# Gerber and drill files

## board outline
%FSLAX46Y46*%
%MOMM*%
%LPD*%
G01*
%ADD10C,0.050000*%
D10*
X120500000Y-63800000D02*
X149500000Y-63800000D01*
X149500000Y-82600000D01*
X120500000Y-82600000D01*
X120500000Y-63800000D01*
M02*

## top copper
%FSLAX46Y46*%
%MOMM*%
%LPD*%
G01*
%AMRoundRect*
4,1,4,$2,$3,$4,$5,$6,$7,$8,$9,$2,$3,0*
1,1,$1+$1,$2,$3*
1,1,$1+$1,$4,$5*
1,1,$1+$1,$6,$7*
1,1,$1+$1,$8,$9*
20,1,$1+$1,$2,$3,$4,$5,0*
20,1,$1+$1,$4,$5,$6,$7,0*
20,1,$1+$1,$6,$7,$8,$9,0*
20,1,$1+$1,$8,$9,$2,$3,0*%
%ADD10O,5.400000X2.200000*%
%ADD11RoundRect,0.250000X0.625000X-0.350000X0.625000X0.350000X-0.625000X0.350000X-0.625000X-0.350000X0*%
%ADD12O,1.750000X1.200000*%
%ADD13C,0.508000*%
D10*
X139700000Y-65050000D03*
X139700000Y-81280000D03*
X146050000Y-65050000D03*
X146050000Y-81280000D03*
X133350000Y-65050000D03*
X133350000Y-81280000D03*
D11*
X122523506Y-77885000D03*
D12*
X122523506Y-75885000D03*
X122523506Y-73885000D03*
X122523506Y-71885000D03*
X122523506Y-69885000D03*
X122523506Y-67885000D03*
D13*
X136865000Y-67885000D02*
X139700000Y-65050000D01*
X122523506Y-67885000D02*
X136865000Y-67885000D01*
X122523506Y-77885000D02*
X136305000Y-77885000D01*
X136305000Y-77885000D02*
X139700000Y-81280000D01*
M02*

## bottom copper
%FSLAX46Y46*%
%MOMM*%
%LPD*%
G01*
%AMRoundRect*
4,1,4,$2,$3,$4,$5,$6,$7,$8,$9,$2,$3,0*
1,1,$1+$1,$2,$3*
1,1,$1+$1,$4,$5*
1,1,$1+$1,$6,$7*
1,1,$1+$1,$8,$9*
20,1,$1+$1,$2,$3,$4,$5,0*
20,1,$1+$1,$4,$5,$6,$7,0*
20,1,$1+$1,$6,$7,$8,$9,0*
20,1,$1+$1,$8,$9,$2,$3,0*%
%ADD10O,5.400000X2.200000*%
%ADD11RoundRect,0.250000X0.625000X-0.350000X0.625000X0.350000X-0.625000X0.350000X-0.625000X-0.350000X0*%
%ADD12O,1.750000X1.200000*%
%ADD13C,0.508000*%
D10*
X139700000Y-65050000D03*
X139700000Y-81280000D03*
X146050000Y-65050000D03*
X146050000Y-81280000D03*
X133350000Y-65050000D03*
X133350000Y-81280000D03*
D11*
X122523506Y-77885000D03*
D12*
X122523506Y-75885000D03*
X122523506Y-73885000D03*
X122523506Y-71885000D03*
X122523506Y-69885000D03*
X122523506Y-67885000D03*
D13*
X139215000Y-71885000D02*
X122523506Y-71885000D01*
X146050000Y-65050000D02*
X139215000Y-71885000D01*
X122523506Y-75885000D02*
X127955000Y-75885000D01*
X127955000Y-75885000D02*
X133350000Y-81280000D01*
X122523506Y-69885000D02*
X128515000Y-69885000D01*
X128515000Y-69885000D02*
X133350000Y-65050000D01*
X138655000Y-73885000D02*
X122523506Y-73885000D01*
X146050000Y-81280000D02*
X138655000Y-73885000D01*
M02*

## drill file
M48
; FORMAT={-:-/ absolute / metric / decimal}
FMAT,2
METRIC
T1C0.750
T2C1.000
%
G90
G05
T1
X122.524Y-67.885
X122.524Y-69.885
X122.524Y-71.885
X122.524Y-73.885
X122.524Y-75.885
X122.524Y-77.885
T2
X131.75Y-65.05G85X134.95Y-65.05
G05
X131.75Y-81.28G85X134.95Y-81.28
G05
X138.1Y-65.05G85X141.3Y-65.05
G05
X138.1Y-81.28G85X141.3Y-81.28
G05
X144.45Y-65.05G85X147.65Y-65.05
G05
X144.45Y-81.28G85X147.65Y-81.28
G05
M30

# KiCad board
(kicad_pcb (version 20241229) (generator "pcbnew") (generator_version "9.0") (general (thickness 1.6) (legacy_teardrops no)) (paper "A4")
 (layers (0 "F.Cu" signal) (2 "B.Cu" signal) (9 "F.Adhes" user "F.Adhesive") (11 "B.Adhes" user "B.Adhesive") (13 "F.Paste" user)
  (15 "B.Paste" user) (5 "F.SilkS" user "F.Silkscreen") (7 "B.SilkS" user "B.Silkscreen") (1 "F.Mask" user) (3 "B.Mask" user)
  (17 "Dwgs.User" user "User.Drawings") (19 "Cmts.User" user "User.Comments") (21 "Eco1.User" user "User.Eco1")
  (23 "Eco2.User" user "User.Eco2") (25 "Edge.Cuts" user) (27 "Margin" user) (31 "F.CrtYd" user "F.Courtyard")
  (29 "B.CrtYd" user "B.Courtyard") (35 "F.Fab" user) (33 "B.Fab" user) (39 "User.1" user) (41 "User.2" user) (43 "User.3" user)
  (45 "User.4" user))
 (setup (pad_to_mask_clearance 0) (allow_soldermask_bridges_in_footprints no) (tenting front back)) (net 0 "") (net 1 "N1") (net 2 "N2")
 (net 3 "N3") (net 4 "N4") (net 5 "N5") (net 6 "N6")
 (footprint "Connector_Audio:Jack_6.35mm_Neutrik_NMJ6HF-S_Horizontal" (layer "F.Cu") (at 133.35 65.05)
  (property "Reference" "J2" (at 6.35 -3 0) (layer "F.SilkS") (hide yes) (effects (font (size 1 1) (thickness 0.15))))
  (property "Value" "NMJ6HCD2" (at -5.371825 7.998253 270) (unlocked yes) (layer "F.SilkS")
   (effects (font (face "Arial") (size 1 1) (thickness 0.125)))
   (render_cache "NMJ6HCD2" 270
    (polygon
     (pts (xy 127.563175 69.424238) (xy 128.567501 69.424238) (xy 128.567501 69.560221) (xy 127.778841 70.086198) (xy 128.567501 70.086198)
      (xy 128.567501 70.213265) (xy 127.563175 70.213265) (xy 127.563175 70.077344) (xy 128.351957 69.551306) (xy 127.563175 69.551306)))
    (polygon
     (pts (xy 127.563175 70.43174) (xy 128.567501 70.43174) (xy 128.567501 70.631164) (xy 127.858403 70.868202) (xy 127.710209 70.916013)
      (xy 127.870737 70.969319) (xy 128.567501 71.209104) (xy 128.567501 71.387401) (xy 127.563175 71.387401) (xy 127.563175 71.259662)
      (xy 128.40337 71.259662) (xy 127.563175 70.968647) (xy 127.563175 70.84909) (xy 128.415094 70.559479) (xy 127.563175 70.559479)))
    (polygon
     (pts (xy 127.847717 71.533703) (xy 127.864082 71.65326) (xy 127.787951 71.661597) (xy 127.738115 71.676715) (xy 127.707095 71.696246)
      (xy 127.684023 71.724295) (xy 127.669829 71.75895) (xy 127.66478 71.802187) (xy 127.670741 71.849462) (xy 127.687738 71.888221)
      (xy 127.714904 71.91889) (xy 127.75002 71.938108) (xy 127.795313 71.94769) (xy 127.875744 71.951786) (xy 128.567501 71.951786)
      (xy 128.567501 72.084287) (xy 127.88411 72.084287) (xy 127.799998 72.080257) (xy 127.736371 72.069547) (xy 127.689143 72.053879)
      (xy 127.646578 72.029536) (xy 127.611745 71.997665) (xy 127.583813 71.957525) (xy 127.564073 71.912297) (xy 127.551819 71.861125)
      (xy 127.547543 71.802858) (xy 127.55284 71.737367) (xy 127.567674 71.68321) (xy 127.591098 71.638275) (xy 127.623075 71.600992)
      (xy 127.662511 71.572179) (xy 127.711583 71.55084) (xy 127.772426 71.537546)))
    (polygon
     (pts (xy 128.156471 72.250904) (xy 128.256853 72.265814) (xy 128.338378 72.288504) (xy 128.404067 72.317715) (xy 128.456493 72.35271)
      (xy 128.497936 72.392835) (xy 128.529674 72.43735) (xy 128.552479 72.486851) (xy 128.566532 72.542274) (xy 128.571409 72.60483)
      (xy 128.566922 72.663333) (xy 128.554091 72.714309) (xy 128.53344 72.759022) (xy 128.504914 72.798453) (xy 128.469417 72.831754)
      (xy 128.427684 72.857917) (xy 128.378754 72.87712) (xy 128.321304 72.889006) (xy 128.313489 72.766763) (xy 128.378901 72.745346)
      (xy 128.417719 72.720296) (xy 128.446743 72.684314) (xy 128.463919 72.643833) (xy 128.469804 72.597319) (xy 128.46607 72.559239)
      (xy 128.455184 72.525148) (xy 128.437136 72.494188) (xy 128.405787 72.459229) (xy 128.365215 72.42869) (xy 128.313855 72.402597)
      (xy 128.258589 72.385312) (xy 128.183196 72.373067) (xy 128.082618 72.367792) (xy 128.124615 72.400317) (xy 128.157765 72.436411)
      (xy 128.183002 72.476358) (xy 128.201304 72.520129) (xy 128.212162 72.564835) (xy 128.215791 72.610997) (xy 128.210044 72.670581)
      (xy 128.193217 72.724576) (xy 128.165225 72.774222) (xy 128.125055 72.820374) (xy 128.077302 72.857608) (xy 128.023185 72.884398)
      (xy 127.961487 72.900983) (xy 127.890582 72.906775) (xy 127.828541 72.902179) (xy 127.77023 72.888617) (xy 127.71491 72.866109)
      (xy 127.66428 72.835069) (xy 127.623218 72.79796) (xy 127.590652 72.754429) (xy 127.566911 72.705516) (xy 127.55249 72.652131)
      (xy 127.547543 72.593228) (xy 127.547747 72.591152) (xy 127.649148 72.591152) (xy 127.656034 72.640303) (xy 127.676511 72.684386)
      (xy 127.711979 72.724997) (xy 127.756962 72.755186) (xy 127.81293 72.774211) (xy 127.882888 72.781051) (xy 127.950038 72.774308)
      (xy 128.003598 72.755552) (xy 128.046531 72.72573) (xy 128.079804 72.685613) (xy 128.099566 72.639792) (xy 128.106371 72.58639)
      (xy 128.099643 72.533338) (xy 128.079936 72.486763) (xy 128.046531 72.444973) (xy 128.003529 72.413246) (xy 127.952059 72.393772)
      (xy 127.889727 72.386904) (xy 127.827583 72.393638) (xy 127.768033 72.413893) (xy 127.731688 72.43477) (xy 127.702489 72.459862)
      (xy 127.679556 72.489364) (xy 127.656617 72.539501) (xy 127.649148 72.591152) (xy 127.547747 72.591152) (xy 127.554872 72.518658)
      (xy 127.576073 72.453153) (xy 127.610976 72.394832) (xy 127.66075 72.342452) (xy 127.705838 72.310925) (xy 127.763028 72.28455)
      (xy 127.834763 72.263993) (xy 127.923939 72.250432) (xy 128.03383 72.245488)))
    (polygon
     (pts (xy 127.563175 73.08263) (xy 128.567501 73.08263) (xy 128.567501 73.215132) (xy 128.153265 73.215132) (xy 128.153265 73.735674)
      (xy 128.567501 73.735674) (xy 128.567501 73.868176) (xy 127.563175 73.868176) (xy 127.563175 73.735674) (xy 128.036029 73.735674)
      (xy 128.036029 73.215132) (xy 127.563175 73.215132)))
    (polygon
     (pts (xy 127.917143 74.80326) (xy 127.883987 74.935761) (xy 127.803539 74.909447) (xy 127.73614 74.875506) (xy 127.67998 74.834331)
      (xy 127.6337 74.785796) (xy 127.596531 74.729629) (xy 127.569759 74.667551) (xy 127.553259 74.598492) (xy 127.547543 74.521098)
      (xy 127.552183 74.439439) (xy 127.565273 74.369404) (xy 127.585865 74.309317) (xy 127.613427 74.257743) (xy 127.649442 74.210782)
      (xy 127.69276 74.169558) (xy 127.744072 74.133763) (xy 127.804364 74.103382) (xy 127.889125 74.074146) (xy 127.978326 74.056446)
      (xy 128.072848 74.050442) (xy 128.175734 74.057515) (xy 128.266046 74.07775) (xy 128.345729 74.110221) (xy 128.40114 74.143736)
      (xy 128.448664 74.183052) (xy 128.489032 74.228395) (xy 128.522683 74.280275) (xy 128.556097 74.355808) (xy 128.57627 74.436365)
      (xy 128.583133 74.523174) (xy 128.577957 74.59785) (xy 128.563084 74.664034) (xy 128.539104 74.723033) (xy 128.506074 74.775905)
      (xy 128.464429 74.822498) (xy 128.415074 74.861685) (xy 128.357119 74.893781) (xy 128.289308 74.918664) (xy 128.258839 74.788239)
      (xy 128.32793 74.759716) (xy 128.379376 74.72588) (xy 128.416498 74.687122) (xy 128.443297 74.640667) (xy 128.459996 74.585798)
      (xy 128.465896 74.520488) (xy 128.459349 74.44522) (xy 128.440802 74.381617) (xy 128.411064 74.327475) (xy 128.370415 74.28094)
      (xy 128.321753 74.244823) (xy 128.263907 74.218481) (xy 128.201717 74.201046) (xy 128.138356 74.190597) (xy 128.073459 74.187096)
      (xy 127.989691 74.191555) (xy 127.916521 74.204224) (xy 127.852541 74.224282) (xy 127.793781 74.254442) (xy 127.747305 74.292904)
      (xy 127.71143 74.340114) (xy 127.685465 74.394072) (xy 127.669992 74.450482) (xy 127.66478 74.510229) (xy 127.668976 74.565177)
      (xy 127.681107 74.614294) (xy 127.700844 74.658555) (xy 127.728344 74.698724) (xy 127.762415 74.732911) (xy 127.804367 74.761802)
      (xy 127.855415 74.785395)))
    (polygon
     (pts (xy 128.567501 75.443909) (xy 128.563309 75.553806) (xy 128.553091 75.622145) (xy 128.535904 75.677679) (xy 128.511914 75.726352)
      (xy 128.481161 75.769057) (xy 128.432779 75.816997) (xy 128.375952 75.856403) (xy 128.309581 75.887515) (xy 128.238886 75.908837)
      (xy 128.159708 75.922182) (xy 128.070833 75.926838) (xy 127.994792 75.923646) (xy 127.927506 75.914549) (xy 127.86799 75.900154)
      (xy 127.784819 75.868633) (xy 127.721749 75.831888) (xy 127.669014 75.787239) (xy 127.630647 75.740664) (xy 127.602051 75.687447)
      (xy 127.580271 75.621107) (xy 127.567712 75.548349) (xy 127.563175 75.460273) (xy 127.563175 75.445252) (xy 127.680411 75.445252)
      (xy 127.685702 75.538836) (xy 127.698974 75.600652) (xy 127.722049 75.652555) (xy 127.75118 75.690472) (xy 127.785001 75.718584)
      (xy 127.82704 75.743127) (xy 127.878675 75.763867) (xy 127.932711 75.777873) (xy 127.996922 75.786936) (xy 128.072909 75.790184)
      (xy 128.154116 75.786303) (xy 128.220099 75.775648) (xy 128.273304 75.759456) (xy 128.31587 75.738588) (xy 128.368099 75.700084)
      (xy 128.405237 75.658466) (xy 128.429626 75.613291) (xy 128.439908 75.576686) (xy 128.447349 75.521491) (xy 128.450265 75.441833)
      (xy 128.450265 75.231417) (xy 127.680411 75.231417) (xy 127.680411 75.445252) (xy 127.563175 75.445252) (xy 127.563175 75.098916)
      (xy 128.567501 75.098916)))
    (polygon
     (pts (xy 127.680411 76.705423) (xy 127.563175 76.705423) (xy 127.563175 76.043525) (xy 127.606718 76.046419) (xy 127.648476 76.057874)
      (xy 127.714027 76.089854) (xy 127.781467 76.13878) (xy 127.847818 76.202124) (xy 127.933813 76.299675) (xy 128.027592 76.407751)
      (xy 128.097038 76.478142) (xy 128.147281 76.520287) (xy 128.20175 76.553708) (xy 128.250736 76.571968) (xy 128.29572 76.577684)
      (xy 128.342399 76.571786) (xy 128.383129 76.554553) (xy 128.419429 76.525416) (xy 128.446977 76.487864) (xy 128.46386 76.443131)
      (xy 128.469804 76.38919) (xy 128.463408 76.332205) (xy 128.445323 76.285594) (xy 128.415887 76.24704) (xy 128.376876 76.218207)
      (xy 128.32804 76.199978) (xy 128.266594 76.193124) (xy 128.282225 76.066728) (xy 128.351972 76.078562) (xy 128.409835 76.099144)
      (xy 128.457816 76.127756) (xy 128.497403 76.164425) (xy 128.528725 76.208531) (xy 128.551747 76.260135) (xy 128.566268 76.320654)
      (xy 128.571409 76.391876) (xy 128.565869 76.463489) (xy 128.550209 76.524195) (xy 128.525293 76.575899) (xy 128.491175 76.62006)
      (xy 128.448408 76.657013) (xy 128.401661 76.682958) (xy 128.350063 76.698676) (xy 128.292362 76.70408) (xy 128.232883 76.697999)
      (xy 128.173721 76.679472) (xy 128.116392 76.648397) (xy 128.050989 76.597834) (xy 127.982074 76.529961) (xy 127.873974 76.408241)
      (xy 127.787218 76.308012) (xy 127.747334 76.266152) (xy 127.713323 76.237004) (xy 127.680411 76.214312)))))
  (pad "R" thru_hole oval (at 6.35 0) (size 5.4 2.2) (drill oval 4.2 1) (layers "*.Cu" "*.Mask") (remove_unused_layers no) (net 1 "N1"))
  (pad "RN" thru_hole oval (at 6.35 16.23) (size 5.4 2.2) (drill oval 4.2 1) (layers "*.Cu" "*.Mask") (remove_unused_layers no) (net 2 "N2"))
  (pad "S" thru_hole oval (at 12.7 0) (size 5.4 2.2) (drill oval 4.2 1) (layers "*.Cu" "*.Mask") (remove_unused_layers no) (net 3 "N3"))
  (pad "SN" thru_hole oval (at 12.7 16.23) (size 5.4 2.2) (drill oval 4.2 1) (layers "*.Cu" "*.Mask") (remove_unused_layers no) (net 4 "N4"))
  (pad "T" thru_hole oval (at 0 0) (size 5.4 2.2) (drill oval 4.2 1) (layers "*.Cu" "*.Mask") (remove_unused_layers no) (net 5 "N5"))
  (pad "TN" thru_hole oval (at 0 16.23) (size 5.4 2.2) (drill oval 4.2 1) (layers "*.Cu" "*.Mask") (remove_unused_layers no) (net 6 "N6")))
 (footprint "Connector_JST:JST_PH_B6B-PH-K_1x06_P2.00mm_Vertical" (layer "F.Cu") (at 122.523506 77.885 90)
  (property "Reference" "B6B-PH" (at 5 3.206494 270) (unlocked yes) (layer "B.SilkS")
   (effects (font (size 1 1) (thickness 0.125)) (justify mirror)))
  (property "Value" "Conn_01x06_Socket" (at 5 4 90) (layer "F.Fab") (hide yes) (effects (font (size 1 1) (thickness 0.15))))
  (pad "1" thru_hole roundrect (at 0 0 90) (size 1.2 1.75) (drill 0.75) (layers "*.Cu" "*.Mask") (remove_unused_layers no)
   (roundrect_rratio 0.208333) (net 2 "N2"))
  (pad "2" thru_hole oval (at 2 0 90) (size 1.2 1.75) (drill 0.75) (layers "*.Cu" "*.Mask") (remove_unused_layers no) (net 6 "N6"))
  (pad "3" thru_hole oval (at 4 0 90) (size 1.2 1.75) (drill 0.75) (layers "*.Cu" "*.Mask") (remove_unused_layers no) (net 4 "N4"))
  (pad "4" thru_hole oval (at 6 0 90) (size 1.2 1.75) (drill 0.75) (layers "*.Cu" "*.Mask") (remove_unused_layers no) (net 3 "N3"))
  (pad "5" thru_hole oval (at 8 0 90) (size 1.2 1.75) (drill 0.75) (layers "*.Cu" "*.Mask") (remove_unused_layers no) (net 5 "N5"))
  (pad "6" thru_hole oval (at 10 0 90) (size 1.2 1.75) (drill 0.75) (layers "*.Cu" "*.Mask") (remove_unused_layers no) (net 1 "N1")))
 (gr_rect (start 120.5 63.8) (end 149.5 82.6) (stroke (width 0.05) (type solid)) (fill no) (layer "Edge.Cuts"))
 (segment (start 139.215 71.885) (end 122.523506 71.885) (width 0.508) (layer "B.Cu") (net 3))
 (segment (start 146.05 65.05) (end 139.215 71.885) (width 0.508) (layer "B.Cu") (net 3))
 (segment (start 136.865 67.885) (end 139.7 65.05) (width 0.508) (layer "F.Cu") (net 1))
 (segment (start 122.523506 67.885) (end 136.865 67.885) (width 0.508) (layer "F.Cu") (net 1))
 (segment (start 122.523506 75.885) (end 127.955 75.885) (width 0.508) (layer "B.Cu") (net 6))
 (segment (start 127.955 75.885) (end 133.35 81.28) (width 0.508) (layer "B.Cu") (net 6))
 (segment (start 122.523506 77.885) (end 136.305 77.885) (width 0.508) (layer "F.Cu") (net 2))
 (segment (start 136.305 77.885) (end 139.7 81.28) (width 0.508) (layer "F.Cu") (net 2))
 (segment (start 122.523506 69.885) (end 128.515 69.885) (width 0.508) (layer "B.Cu") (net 5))
 (segment (start 128.515 69.885) (end 133.35 65.05) (width 0.508) (layer "B.Cu") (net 5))
 (segment (start 138.655 73.885) (end 122.523506 73.885) (width 0.508) (layer "B.Cu") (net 4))
 (segment (start 146.05 81.28) (end 138.655 73.885) (width 0.508) (layer "B.Cu") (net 4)))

